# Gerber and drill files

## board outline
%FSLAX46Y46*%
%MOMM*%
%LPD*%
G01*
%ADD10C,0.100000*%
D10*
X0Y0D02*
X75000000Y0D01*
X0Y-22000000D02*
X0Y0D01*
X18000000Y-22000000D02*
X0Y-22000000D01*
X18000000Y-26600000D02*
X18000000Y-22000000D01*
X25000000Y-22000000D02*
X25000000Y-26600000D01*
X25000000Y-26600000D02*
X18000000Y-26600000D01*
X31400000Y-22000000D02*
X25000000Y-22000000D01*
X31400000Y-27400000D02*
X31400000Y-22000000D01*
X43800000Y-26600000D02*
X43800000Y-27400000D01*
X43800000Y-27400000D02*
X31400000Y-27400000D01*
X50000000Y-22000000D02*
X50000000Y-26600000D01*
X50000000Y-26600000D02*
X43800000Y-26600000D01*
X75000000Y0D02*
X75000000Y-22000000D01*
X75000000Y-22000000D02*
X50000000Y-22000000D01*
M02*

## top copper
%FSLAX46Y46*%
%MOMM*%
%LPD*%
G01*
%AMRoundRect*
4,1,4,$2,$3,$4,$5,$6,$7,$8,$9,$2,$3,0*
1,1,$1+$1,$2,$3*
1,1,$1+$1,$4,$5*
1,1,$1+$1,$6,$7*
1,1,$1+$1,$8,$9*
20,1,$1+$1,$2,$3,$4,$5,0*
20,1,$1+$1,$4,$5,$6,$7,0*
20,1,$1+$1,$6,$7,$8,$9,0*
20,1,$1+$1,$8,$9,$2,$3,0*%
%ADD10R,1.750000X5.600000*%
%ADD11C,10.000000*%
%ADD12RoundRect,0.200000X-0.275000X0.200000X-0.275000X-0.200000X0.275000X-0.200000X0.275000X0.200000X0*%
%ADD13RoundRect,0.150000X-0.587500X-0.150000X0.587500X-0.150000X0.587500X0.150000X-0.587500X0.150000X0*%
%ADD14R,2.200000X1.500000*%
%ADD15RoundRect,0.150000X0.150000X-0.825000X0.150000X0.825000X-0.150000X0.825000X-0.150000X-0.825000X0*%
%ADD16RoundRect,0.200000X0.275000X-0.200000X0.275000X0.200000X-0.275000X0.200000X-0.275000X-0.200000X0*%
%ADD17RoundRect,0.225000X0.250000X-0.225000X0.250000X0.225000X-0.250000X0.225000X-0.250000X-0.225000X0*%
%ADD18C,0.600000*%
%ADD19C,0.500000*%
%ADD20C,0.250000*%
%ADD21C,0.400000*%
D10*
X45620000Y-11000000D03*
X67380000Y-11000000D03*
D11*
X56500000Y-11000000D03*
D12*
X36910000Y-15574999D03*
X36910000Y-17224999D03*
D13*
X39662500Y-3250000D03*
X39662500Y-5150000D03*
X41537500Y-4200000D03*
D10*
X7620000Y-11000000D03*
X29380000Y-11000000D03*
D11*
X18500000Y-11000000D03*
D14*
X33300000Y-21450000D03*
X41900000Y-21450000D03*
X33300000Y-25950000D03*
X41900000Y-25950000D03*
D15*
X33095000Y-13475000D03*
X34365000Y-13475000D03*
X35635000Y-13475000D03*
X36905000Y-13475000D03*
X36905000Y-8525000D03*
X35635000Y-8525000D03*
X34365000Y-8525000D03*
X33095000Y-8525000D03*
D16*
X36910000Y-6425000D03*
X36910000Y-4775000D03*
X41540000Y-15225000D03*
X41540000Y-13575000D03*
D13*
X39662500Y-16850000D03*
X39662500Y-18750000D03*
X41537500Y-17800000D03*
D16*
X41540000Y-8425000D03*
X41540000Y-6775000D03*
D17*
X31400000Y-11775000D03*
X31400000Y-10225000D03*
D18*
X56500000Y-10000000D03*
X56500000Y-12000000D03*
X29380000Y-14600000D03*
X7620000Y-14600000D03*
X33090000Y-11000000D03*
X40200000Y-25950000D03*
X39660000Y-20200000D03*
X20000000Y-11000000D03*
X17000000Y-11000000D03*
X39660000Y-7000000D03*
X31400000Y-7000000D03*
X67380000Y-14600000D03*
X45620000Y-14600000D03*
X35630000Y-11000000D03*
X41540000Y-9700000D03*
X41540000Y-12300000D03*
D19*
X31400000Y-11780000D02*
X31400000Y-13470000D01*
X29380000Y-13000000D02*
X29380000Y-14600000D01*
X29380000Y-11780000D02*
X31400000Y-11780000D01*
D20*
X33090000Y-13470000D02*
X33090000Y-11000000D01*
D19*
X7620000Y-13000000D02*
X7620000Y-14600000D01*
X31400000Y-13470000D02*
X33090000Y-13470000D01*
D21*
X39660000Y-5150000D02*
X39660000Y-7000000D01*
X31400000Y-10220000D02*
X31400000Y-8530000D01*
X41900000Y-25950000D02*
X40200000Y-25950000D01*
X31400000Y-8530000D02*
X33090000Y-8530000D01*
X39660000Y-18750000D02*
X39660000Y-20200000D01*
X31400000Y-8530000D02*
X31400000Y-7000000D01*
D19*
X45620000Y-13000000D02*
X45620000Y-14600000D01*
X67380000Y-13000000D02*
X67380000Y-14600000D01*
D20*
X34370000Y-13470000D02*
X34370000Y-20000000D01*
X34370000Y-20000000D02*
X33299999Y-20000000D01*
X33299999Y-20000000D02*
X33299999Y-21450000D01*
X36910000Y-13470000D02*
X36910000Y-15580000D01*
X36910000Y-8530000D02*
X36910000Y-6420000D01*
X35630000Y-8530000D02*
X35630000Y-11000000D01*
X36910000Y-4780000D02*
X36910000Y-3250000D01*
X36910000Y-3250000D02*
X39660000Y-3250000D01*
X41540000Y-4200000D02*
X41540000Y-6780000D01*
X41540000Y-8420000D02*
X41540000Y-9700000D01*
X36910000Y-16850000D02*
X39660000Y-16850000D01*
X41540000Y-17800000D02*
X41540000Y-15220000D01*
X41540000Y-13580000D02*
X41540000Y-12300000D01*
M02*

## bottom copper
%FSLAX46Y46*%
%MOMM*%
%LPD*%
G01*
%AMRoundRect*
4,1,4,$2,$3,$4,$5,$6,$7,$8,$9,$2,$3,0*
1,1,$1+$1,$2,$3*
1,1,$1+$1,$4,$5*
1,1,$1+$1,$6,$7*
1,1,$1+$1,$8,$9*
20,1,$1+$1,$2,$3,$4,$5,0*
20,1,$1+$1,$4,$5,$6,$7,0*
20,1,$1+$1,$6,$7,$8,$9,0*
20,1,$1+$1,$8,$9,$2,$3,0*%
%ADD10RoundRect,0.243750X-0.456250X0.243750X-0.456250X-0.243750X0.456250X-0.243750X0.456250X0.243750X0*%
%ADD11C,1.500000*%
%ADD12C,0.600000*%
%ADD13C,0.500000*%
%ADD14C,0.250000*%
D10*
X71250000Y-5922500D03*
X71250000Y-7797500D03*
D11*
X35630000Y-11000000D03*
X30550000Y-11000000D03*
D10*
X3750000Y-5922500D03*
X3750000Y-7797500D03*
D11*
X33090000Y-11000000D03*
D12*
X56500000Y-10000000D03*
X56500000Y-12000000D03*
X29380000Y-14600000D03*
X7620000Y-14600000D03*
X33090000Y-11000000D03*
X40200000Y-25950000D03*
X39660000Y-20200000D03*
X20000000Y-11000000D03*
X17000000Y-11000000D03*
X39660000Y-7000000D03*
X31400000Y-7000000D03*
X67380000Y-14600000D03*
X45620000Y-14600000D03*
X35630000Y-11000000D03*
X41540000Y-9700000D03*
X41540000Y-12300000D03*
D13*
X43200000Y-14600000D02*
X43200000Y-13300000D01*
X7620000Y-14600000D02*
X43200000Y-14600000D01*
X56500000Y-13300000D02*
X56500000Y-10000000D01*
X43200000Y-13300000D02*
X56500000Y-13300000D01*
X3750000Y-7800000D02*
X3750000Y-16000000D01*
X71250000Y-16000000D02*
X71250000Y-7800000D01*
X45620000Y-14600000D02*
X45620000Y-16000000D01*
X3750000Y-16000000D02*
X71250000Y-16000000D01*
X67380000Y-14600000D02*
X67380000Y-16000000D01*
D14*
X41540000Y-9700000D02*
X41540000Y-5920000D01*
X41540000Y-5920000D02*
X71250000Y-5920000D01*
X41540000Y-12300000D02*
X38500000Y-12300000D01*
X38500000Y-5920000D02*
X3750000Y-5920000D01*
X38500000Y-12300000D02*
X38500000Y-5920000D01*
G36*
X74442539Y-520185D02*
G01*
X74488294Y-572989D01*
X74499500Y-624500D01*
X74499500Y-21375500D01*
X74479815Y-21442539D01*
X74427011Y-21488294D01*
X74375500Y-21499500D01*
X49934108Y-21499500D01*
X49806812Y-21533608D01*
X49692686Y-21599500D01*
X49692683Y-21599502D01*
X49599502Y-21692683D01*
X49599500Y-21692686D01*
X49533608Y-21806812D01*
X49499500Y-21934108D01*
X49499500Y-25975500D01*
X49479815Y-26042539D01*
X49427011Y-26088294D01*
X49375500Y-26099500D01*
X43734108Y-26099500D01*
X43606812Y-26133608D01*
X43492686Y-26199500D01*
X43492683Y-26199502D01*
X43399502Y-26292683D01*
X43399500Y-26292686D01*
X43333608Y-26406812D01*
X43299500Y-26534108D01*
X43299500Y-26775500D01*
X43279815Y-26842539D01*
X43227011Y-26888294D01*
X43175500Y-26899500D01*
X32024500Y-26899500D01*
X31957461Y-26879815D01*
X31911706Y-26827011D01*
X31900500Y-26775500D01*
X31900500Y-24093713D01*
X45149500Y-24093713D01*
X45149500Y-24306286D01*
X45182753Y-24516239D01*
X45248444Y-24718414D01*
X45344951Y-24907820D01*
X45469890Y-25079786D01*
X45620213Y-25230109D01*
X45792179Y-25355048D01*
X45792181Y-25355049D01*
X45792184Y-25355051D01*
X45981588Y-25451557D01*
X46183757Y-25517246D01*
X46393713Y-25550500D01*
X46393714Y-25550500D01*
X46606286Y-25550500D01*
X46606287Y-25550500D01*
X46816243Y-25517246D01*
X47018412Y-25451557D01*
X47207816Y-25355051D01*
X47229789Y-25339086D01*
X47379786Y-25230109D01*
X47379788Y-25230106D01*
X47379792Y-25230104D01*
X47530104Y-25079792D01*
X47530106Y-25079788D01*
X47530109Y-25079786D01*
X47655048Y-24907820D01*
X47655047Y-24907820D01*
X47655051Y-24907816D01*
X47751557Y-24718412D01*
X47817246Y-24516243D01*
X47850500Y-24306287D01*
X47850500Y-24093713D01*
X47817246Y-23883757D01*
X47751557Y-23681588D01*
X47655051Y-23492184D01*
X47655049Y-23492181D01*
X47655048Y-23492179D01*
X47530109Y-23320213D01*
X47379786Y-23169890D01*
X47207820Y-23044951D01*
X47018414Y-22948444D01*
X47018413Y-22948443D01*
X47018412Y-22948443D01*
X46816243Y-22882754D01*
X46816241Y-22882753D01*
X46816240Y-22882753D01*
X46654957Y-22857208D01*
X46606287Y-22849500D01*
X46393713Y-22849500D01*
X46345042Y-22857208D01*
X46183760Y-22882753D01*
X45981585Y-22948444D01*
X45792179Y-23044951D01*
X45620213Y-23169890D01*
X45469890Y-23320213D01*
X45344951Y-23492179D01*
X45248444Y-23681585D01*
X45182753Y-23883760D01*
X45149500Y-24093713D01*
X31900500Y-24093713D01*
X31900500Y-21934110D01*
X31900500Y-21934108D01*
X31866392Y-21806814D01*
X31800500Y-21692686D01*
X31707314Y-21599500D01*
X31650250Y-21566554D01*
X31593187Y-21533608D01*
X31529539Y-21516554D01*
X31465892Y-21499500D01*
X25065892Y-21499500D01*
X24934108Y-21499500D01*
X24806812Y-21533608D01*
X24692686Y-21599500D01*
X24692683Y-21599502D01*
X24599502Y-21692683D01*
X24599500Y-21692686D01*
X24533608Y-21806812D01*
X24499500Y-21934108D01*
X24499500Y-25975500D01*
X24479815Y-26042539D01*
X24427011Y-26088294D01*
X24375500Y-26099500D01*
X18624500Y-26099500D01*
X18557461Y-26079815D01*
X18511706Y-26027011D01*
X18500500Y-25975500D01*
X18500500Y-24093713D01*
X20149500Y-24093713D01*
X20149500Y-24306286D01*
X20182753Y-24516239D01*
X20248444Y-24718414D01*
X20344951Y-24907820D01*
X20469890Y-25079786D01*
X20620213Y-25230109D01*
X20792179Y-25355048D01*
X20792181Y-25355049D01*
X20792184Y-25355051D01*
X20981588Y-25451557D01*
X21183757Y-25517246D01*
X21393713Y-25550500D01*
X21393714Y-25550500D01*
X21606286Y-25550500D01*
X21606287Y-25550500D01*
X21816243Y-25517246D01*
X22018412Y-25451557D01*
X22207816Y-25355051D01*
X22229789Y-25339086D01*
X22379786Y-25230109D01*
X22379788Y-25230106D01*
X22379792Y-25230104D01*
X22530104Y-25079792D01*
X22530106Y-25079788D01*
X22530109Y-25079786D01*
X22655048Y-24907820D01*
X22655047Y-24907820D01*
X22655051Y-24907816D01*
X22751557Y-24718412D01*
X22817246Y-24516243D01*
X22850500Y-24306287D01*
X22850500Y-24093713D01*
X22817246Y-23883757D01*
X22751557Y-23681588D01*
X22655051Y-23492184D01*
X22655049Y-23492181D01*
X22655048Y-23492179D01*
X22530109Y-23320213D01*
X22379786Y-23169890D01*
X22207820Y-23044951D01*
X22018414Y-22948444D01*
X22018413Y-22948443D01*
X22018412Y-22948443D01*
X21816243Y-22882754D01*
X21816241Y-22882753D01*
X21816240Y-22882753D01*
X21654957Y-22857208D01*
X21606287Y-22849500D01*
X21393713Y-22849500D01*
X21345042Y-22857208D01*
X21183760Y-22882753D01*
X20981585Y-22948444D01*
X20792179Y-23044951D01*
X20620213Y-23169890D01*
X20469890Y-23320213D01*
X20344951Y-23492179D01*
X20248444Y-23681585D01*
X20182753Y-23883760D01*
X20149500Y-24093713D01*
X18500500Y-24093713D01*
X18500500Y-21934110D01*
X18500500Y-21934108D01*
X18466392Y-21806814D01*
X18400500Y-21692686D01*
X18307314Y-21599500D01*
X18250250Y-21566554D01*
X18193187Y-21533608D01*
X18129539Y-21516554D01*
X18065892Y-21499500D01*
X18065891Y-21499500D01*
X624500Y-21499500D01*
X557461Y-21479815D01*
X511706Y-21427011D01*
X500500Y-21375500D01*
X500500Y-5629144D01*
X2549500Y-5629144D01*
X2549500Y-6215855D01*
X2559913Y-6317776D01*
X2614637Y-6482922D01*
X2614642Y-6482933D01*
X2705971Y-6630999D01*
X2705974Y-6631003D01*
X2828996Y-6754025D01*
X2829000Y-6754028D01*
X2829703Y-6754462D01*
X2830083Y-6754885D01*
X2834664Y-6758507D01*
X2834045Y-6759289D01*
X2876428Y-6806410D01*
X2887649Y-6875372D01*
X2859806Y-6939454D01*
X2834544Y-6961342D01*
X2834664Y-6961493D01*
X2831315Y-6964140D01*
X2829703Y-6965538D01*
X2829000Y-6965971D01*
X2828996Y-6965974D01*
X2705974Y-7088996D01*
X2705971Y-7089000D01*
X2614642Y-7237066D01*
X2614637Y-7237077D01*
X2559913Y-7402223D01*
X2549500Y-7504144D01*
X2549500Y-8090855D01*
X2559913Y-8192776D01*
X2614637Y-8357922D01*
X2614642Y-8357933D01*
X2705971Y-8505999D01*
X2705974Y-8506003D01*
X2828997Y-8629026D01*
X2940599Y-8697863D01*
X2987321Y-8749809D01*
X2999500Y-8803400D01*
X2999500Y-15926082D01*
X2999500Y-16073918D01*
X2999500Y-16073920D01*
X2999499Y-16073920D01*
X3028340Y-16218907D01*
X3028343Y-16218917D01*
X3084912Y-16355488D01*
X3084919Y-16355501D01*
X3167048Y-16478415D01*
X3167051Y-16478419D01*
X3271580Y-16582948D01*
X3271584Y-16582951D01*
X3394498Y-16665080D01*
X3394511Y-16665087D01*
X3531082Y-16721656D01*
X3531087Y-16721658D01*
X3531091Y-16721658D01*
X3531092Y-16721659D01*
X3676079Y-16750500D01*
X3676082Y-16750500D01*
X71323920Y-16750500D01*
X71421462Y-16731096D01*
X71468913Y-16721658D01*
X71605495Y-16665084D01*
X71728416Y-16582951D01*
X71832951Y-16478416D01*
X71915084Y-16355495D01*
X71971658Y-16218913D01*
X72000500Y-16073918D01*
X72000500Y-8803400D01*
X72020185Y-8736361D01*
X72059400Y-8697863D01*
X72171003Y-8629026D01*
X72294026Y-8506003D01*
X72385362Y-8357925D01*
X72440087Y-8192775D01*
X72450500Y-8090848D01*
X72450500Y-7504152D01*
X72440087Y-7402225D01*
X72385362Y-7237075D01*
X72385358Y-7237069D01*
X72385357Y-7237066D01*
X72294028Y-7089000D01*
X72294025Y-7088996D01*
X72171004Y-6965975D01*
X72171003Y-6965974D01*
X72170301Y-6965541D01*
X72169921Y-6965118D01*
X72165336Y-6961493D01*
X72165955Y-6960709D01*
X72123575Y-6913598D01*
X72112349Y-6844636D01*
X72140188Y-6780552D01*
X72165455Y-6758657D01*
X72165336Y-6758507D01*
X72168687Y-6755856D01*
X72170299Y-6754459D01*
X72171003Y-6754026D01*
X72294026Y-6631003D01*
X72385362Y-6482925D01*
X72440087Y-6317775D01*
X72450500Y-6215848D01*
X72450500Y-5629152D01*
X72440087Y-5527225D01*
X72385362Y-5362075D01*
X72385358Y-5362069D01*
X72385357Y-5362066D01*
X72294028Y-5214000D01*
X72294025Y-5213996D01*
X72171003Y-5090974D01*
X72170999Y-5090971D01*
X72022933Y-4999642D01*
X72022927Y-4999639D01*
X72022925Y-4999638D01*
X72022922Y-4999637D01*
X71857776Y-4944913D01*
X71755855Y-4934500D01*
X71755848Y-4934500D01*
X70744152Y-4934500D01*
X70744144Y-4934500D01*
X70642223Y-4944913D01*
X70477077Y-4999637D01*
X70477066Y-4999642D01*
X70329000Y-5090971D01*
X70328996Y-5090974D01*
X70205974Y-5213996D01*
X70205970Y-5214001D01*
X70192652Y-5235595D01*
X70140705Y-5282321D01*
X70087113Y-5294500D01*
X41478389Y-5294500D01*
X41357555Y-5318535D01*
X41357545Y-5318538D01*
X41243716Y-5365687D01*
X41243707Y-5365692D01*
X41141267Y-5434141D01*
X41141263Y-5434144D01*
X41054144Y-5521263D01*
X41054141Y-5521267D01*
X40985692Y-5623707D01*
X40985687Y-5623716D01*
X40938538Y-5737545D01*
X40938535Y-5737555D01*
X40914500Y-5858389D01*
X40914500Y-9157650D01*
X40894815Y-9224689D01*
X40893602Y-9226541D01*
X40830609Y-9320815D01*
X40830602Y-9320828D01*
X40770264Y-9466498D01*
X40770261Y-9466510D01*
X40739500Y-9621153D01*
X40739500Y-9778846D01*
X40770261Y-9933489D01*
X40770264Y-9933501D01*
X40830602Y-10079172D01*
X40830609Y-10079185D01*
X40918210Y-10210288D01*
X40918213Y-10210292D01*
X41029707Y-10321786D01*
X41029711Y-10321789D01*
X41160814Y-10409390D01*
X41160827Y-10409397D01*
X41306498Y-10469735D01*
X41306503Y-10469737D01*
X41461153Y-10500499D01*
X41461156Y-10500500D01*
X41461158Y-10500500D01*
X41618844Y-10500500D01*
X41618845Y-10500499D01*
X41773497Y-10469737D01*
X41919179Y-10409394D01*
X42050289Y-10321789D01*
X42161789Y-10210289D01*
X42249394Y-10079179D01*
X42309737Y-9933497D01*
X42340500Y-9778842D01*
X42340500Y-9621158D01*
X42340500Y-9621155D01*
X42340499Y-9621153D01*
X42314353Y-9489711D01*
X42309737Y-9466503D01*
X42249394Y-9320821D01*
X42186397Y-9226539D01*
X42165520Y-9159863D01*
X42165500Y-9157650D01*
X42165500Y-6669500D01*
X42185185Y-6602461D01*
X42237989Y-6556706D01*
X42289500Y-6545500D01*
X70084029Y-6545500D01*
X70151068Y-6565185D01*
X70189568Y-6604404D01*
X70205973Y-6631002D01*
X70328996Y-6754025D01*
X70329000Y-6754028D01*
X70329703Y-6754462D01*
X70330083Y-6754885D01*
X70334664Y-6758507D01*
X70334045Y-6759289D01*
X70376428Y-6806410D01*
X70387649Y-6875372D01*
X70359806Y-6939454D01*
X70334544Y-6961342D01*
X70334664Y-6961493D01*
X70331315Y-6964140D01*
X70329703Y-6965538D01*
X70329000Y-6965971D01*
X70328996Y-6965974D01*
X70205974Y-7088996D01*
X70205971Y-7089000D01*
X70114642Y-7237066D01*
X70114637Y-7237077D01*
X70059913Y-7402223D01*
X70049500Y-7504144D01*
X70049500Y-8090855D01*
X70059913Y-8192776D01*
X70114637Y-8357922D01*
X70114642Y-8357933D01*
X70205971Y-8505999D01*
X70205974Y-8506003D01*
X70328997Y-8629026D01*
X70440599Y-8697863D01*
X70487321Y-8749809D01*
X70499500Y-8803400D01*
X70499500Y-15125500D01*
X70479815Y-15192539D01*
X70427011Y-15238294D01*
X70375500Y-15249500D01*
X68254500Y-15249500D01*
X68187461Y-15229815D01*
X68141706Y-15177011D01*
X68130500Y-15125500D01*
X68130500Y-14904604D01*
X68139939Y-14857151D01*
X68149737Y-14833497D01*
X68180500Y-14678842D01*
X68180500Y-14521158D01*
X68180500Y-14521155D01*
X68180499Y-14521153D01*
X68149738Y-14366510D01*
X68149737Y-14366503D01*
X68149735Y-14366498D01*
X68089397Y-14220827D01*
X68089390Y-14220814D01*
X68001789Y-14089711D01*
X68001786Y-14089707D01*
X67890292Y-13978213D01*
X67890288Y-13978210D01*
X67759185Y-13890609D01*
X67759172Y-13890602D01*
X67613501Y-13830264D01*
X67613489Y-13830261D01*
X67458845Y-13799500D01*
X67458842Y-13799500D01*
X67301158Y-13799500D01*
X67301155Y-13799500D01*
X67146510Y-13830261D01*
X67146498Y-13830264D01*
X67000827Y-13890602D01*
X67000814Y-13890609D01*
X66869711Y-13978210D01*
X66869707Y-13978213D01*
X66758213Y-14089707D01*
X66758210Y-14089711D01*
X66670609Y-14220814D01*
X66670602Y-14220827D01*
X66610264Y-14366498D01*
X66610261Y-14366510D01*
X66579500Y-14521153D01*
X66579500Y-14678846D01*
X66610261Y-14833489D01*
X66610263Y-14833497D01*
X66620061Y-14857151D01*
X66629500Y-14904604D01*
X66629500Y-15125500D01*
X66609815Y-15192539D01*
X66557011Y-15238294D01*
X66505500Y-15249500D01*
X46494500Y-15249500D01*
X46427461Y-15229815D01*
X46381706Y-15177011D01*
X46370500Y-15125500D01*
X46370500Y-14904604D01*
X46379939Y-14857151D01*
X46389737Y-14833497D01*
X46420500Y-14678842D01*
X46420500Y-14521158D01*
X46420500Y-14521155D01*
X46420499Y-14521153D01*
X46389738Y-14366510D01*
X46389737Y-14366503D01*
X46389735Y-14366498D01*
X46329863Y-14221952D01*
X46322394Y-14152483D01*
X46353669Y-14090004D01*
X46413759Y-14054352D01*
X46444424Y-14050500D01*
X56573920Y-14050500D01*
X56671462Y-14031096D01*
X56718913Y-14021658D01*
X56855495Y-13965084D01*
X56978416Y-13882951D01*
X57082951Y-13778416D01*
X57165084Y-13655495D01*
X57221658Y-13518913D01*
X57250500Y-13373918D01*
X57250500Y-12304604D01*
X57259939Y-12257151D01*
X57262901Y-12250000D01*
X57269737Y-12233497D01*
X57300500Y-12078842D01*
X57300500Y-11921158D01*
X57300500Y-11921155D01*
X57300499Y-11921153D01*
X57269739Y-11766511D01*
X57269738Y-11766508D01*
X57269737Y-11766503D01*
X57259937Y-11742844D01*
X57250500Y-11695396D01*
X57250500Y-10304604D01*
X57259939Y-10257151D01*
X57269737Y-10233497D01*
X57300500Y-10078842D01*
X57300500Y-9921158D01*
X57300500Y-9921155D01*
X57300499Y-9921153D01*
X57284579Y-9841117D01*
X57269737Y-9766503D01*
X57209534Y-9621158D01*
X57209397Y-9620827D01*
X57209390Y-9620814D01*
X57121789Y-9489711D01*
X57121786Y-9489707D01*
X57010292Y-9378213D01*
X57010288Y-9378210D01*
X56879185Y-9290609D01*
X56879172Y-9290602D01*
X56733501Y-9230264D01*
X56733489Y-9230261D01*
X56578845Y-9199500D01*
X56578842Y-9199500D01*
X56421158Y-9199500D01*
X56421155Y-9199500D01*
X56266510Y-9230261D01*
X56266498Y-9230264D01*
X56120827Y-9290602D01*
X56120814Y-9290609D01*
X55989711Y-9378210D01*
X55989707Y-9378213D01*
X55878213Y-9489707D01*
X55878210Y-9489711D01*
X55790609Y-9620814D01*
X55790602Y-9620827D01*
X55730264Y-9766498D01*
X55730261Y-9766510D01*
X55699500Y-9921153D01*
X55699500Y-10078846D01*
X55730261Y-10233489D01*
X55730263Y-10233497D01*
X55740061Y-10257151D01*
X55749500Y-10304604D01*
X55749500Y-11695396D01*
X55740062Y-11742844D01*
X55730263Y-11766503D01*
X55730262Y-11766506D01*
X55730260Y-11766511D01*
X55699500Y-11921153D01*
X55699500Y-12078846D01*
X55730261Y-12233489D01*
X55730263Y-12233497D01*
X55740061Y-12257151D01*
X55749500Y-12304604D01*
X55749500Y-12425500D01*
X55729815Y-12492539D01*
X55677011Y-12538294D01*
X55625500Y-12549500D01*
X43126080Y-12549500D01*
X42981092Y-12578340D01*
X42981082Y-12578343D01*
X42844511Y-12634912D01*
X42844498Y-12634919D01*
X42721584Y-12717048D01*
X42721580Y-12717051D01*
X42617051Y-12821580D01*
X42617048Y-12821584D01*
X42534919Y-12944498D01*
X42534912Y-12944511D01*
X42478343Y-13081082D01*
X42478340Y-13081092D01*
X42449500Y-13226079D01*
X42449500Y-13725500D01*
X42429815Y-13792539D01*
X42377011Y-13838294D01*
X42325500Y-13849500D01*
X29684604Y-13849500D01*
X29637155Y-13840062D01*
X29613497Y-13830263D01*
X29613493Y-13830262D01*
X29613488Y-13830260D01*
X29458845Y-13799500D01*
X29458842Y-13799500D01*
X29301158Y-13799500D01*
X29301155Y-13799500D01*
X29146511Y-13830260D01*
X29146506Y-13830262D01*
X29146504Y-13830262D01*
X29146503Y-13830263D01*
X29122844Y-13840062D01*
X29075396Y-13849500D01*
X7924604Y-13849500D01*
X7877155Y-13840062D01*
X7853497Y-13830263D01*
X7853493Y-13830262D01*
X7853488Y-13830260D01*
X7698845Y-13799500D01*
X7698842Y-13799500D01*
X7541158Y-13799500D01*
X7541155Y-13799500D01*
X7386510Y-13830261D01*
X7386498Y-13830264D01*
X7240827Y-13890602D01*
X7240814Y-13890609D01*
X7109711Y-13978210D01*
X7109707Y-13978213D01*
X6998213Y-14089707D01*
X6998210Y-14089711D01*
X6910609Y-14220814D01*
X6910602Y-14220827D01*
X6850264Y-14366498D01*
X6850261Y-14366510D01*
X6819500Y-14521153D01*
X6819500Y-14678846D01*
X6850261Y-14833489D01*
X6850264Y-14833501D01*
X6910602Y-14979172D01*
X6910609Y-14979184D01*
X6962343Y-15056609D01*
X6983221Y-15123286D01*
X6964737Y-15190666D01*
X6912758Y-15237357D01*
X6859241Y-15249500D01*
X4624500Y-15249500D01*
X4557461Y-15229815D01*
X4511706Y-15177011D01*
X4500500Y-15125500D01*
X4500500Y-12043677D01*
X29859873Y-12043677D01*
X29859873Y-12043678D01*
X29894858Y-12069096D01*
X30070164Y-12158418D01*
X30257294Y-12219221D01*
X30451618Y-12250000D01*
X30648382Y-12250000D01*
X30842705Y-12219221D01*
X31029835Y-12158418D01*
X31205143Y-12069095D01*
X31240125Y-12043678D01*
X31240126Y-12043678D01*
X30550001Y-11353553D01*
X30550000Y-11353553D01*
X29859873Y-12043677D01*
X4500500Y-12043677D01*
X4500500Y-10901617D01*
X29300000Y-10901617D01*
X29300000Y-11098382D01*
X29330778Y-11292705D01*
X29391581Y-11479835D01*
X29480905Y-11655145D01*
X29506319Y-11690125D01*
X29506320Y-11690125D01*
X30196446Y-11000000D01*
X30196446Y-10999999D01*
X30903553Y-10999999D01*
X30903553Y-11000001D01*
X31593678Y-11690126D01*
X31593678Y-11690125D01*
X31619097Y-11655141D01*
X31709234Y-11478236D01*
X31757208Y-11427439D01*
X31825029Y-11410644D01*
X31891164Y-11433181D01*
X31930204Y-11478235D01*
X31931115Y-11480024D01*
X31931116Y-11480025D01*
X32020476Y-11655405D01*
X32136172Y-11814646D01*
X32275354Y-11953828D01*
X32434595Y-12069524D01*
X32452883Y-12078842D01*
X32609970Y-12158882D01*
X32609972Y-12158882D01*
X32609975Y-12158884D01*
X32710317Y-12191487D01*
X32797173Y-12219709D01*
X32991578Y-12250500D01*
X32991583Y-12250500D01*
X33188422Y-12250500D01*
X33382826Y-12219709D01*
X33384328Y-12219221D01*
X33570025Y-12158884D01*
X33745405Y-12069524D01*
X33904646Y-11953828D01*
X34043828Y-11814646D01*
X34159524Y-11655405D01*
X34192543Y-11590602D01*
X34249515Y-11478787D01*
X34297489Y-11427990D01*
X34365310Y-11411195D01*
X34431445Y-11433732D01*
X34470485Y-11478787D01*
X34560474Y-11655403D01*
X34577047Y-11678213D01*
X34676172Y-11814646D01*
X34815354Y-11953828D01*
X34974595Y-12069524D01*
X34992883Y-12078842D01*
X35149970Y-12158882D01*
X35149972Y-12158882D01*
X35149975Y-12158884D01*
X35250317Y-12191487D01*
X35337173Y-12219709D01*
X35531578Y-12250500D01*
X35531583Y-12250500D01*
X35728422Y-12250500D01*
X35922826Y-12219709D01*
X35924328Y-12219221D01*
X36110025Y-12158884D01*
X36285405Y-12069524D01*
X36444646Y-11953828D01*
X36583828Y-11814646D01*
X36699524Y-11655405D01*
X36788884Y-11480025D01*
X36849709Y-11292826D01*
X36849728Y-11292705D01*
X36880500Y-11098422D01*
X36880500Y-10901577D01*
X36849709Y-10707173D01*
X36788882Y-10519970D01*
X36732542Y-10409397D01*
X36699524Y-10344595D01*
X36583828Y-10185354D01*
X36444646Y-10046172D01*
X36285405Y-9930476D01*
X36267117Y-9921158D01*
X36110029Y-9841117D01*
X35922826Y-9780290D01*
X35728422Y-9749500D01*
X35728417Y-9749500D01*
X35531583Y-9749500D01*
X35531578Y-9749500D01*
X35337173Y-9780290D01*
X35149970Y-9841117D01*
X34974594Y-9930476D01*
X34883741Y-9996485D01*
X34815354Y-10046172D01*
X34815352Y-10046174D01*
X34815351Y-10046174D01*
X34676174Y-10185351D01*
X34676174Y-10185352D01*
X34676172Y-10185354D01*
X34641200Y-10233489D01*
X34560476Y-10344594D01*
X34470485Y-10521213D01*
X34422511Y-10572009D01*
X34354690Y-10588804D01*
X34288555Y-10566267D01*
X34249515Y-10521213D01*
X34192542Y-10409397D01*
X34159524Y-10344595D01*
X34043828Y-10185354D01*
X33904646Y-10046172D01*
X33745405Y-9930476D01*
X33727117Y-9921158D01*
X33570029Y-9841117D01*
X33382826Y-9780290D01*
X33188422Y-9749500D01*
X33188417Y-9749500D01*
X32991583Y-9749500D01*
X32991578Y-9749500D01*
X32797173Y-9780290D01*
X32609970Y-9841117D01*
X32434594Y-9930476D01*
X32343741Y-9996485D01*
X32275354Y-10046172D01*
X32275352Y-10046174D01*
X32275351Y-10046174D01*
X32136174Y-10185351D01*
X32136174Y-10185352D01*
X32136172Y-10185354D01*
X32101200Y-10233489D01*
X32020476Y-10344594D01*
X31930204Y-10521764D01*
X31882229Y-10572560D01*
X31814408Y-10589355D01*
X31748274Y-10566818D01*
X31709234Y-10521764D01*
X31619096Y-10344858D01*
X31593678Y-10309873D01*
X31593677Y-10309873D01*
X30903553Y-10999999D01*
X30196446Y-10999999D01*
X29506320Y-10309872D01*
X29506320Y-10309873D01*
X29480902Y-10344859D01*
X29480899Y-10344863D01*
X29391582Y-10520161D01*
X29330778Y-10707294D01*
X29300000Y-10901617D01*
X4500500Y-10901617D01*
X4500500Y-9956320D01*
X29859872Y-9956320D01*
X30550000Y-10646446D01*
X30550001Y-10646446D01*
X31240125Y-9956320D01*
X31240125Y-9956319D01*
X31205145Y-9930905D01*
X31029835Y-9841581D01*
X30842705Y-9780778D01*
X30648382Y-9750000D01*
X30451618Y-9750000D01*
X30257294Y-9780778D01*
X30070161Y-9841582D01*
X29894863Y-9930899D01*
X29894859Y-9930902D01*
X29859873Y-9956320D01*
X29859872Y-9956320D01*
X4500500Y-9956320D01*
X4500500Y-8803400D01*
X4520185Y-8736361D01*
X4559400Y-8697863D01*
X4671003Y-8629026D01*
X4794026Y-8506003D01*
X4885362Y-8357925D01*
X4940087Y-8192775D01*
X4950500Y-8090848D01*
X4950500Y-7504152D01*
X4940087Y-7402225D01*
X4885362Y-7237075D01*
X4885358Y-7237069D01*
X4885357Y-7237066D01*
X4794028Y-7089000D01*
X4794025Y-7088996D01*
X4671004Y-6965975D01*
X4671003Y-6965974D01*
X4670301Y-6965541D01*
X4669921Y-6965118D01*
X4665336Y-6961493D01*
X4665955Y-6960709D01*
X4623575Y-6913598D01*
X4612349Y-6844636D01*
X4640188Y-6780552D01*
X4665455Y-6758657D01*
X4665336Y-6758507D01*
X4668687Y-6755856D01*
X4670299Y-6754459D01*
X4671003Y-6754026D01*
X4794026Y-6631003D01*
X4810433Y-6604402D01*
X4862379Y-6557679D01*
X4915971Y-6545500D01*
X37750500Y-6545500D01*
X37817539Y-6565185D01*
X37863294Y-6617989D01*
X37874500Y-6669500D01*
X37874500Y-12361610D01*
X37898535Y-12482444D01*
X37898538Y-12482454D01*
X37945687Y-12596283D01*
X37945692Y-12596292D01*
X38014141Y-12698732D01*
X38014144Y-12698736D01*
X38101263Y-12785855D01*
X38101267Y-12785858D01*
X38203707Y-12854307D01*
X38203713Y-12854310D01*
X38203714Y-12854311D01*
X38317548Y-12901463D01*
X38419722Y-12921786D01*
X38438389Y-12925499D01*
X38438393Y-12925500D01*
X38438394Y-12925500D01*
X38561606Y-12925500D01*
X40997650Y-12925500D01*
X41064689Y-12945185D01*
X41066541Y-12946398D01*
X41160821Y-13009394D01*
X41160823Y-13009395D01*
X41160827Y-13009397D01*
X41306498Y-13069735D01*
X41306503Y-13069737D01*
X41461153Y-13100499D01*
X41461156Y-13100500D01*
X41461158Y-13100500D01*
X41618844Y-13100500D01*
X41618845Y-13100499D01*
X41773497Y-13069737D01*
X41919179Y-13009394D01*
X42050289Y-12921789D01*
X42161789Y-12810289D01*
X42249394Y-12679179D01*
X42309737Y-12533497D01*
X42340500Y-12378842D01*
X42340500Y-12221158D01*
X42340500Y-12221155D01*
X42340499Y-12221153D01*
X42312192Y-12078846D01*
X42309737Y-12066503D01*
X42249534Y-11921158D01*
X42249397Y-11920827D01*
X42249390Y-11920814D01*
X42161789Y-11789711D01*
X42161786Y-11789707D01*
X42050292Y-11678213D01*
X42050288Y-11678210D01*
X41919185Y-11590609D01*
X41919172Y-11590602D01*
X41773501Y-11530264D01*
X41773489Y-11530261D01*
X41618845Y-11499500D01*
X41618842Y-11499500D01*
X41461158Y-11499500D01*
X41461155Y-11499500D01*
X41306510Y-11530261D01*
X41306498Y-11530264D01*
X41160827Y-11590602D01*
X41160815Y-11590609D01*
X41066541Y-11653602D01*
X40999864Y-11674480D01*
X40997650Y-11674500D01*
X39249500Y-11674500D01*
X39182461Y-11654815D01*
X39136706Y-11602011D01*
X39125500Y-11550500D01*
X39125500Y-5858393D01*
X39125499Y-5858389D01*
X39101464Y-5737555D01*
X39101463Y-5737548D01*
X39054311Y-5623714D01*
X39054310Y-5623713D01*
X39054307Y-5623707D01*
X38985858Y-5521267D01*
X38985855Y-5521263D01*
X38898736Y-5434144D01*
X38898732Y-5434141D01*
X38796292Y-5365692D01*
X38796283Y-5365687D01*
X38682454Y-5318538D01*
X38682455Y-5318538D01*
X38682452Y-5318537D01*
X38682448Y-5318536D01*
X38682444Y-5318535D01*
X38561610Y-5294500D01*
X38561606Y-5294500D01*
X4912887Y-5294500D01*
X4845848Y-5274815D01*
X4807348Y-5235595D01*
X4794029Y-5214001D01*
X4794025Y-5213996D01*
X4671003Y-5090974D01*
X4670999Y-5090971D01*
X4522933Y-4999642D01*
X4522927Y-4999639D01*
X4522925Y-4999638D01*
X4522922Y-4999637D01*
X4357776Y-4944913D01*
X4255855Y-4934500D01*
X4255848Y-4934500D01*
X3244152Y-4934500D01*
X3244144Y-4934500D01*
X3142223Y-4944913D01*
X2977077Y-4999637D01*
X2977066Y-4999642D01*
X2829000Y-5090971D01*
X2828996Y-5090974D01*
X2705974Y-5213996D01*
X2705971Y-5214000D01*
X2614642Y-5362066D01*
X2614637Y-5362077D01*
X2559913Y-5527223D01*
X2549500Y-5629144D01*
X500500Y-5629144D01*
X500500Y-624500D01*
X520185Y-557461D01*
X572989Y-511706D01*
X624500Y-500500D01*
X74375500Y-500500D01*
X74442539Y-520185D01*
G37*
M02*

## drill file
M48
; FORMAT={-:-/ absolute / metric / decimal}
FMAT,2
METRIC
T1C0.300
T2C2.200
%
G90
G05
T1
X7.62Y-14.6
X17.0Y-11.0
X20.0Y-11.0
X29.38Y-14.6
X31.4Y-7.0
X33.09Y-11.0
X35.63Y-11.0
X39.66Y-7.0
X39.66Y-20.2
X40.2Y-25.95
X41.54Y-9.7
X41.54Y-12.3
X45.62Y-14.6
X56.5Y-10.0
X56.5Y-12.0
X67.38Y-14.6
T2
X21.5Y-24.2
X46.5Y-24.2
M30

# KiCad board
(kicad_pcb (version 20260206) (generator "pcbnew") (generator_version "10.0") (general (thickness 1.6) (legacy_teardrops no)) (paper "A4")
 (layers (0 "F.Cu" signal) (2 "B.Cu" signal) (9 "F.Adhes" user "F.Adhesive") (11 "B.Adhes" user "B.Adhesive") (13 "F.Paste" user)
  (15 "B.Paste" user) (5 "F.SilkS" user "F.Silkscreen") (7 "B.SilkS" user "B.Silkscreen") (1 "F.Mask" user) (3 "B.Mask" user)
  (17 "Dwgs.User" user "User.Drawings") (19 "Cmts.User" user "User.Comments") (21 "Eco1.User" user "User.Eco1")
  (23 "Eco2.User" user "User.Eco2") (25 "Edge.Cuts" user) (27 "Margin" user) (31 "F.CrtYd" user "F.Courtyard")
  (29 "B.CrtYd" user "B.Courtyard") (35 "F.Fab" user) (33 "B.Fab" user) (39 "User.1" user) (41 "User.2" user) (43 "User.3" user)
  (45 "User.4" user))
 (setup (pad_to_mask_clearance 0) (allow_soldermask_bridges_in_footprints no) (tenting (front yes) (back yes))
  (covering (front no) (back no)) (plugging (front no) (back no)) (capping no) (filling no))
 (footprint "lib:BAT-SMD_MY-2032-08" (layer "F.Cu") (at 56.5 11)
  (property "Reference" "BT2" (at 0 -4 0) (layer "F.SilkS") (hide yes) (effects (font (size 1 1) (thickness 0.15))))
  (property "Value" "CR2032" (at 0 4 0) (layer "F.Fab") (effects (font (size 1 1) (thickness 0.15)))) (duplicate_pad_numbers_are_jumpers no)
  (pad "1" smd rect (at -10.88 0) (size 1.75 5.6) (layers "F.Cu" "F.Mask" "F.Paste") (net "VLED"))
  (pad "1" smd rect (at 10.88 0) (size 1.75 5.6) (layers "F.Cu" "F.Mask" "F.Paste") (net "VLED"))
  (pad "2" smd circle (at 0 0) (size 10 10) (layers "F.Cu" "F.Mask" "F.Paste") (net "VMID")))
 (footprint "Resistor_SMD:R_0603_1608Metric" (layer "F.Cu") (at 36.91 16.399999 -90)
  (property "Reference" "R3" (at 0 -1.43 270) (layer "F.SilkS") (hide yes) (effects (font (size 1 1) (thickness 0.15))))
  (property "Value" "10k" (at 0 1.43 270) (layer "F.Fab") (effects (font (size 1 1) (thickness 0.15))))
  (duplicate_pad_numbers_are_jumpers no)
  (pad "1" smd roundrect (at -0.825 0 270) (size 0.8 0.95) (layers "F.Cu" "F.Mask" "F.Paste") (roundrect_rratio 0.25) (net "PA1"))
  (pad "2" smd roundrect (at 0.825 0 270) (size 0.8 0.95) (layers "F.Cu" "F.Mask" "F.Paste") (roundrect_rratio 0.25) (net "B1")))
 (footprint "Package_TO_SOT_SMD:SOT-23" (layer "F.Cu") (at 40.6 4.2)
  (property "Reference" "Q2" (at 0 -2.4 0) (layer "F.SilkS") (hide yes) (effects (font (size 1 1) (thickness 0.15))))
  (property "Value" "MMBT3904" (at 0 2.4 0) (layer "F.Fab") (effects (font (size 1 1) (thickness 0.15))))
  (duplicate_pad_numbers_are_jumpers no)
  (pad "1" smd roundrect (at -0.9375 -0.95) (size 1.475 0.6) (layers "F.Cu" "F.Mask" "F.Paste") (roundrect_rratio 0.25) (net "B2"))
  (pad "2" smd roundrect (at -0.9375 0.95) (size 1.475 0.6) (layers "F.Cu" "F.Mask" "F.Paste") (roundrect_rratio 0.25) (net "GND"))
  (pad "3" smd roundrect (at 0.9375 0) (size 1.475 0.6) (layers "F.Cu" "F.Mask" "F.Paste") (roundrect_rratio 0.25) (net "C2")))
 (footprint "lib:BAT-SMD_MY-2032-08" (layer "F.Cu") (at 18.5 11)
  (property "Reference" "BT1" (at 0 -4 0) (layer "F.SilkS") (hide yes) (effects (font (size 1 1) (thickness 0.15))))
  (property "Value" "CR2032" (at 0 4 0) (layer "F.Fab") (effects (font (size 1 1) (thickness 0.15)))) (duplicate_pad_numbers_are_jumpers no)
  (pad "1" smd rect (at -10.88 0) (size 1.75 5.6) (layers "F.Cu" "F.Mask" "F.Paste") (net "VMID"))
  (pad "1" smd rect (at 10.88 0) (size 1.75 5.6) (layers "F.Cu" "F.Mask" "F.Paste") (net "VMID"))
  (pad "2" smd circle (at 0 0) (size 10 10) (layers "F.Cu" "F.Mask" "F.Paste") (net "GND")))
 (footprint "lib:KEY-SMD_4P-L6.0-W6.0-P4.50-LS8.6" (layer "F.Cu") (at 37.6 23.7)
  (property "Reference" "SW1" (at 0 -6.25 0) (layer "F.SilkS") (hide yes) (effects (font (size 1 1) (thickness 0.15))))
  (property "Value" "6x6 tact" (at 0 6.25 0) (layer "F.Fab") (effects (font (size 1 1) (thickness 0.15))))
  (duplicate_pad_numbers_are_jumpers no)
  (pad "1" smd rect (at -4.3 -2.25) (size 2.2 1.5) (layers "F.Cu" "F.Mask" "F.Paste") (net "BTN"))
  (pad "2" smd rect (at 4.3 -2.25) (size 2.2 1.5) (layers "F.Cu" "F.Mask" "F.Paste"))
  (pad "3" smd rect (at -4.3 2.25) (size 2.2 1.5) (layers "F.Cu" "F.Mask" "F.Paste"))
  (pad "4" smd rect (at 4.3 2.25) (size 2.2 1.5) (layers "F.Cu" "F.Mask" "F.Paste") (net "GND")))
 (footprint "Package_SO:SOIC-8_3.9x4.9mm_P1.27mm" (layer "F.Cu") (at 35 11 90)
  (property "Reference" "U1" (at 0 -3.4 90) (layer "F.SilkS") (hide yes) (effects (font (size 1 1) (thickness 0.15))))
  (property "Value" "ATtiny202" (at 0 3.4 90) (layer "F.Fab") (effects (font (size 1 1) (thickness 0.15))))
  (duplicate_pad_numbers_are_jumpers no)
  (pad "1" smd roundrect (at -2.475 -1.905 90) (size 1.95 0.6) (layers "F.Cu" "F.Mask" "F.Paste") (roundrect_rratio 0.25) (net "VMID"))
  (pad "2" smd roundrect (at -2.475 -0.635 90) (size 1.95 0.6) (layers "F.Cu" "F.Mask" "F.Paste") (roundrect_rratio 0.25) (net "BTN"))
  (pad "3" smd roundrect (at -2.475 0.635 90) (size 1.95 0.6) (layers "F.Cu" "F.Mask" "F.Paste") (roundrect_rratio 0.25))
  (pad "4" smd roundrect (at -2.475 1.905 90) (size 1.95 0.6) (layers "F.Cu" "F.Mask" "F.Paste") (roundrect_rratio 0.25) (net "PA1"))
  (pad "5" smd roundrect (at 2.475 1.905 90) (size 1.95 0.6) (layers "F.Cu" "F.Mask" "F.Paste") (roundrect_rratio 0.25) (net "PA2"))
  (pad "6" smd roundrect (at 2.475 0.635 90) (size 1.95 0.6) (layers "F.Cu" "F.Mask" "F.Paste") (roundrect_rratio 0.25) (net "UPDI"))
  (pad "7" smd roundrect (at 2.475 -0.635 90) (size 1.95 0.6) (layers "F.Cu" "F.Mask" "F.Paste") (roundrect_rratio 0.25))
  (pad "8" smd roundrect (at 2.475 -1.905 90) (size 1.95 0.6) (layers "F.Cu" "F.Mask" "F.Paste") (roundrect_rratio 0.25) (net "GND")))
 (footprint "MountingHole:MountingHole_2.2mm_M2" (layer "F.Cu") (at 21.5 24.2)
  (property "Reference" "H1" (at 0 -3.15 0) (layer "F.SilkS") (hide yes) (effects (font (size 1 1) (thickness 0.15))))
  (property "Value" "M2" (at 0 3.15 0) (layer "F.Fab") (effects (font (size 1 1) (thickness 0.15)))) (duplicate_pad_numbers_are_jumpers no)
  (pad "" np_thru_hole circle (at 0 0) (size 2.2 2.2) (drill 2.2) (layers "*.Cu" "*.Mask")))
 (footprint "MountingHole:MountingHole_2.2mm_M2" (layer "F.Cu") (at 46.5 24.2)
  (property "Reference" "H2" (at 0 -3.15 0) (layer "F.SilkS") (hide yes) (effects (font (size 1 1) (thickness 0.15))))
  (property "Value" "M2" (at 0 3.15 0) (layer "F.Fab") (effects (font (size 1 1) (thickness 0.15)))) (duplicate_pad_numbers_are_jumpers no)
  (pad "" np_thru_hole circle (at 0 0) (size 2.2 2.2) (drill 2.2) (layers "*.Cu" "*.Mask")))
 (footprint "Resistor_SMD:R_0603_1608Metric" (layer "F.Cu") (at 36.91 5.6 90)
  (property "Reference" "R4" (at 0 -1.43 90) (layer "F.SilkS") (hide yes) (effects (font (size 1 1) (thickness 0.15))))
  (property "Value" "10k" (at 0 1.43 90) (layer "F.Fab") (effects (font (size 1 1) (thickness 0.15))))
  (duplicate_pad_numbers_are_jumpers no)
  (pad "1" smd roundrect (at -0.825 0 90) (size 0.8 0.95) (layers "F.Cu" "F.Mask" "F.Paste") (roundrect_rratio 0.25) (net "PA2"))
  (pad "2" smd roundrect (at 0.825 0 90) (size 0.8 0.95) (layers "F.Cu" "F.Mask" "F.Paste") (roundrect_rratio 0.25) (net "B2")))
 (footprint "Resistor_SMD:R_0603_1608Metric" (layer "F.Cu") (at 41.54 14.4 90)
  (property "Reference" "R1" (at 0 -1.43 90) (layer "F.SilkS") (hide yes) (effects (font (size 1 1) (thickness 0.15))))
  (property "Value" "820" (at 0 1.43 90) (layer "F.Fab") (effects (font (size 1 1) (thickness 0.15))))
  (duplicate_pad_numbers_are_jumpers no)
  (pad "1" smd roundrect (at -0.825 0 90) (size 0.8 0.95) (layers "F.Cu" "F.Mask" "F.Paste") (roundrect_rratio 0.25) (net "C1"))
  (pad "2" smd roundrect (at 0.825 0 90) (size 0.8 0.95) (layers "F.Cu" "F.Mask" "F.Paste") (roundrect_rratio 0.25) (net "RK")))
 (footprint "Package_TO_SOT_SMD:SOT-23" (layer "F.Cu") (at 40.6 17.8)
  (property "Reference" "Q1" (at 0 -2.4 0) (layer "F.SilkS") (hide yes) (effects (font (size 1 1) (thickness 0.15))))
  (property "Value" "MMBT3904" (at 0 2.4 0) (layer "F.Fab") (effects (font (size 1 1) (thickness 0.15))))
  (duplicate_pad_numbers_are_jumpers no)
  (pad "1" smd roundrect (at -0.9375 -0.95) (size 1.475 0.6) (layers "F.Cu" "F.Mask" "F.Paste") (roundrect_rratio 0.25) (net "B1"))
  (pad "2" smd roundrect (at -0.9375 0.95) (size 1.475 0.6) (layers "F.Cu" "F.Mask" "F.Paste") (roundrect_rratio 0.25) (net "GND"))
  (pad "3" smd roundrect (at 0.9375 0) (size 1.475 0.6) (layers "F.Cu" "F.Mask" "F.Paste") (roundrect_rratio 0.25) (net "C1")))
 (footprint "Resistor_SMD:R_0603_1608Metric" (layer "F.Cu") (at 41.54 7.6 90)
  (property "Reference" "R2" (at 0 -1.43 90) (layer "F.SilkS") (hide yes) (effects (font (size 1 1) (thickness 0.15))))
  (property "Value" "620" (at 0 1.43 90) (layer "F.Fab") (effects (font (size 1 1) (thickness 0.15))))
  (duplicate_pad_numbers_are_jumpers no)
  (pad "1" smd roundrect (at -0.825 0 90) (size 0.8 0.95) (layers "F.Cu" "F.Mask" "F.Paste") (roundrect_rratio 0.25) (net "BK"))
  (pad "2" smd roundrect (at 0.825 0 90) (size 0.8 0.95) (layers "F.Cu" "F.Mask" "F.Paste") (roundrect_rratio 0.25) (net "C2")))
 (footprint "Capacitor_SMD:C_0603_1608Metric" (layer "F.Cu") (at 31.4 11 90)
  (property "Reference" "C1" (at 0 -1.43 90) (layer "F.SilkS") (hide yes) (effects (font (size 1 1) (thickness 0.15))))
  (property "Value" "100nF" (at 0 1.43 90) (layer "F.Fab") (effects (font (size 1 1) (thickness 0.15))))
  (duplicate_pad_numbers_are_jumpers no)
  (pad "1" smd roundrect (at -0.775 0 90) (size 0.9 0.95) (layers "F.Cu" "F.Mask" "F.Paste") (roundrect_rratio 0.25) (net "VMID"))
  (pad "2" smd roundrect (at 0.775 0 90) (size 0.9 0.95) (layers "F.Cu" "F.Mask" "F.Paste") (roundrect_rratio 0.25) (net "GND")))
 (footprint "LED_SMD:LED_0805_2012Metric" (layer "B.Cu") (at 71.25 6.86 -90)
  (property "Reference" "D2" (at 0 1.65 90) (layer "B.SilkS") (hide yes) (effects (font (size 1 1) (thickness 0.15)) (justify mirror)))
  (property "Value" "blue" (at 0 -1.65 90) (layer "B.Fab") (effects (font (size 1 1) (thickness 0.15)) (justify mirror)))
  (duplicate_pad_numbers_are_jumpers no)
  (pad "1" smd roundrect (at -0.9375 0 270) (size 0.975 1.4) (layers "B.Cu" "B.Mask" "B.Paste") (roundrect_rratio 0.25) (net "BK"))
  (pad "2" smd roundrect (at 0.9375 0 270) (size 0.975 1.4) (layers "B.Cu" "B.Mask" "B.Paste") (roundrect_rratio 0.25) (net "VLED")))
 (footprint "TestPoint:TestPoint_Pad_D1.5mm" (layer "B.Cu") (at 35.63 11)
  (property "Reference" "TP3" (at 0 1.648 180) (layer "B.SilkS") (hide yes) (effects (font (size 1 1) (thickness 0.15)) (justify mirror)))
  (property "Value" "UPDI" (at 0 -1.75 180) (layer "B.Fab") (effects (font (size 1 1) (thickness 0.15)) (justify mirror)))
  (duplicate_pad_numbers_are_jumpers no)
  (pad "1" smd circle (at 0 0) (size 1.5 1.5) (layers "B.Cu" "B.Mask") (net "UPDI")))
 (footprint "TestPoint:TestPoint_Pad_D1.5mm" (layer "B.Cu") (at 30.55 11)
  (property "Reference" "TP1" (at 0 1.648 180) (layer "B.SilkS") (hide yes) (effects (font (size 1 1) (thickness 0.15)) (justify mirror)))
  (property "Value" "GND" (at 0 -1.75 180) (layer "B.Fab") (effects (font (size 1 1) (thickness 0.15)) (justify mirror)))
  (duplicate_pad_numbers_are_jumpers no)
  (pad "1" smd circle (at 0 0) (size 1.5 1.5) (layers "B.Cu" "B.Mask") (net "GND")))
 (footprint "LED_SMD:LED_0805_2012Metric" (layer "B.Cu") (at 3.75 6.86 -90)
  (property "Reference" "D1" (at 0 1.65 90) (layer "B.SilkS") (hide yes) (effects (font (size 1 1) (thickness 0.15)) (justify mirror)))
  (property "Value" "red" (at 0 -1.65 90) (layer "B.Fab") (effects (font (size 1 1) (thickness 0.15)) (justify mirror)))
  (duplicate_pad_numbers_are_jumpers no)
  (pad "1" smd roundrect (at -0.9375 0 270) (size 0.975 1.4) (layers "B.Cu" "B.Mask" "B.Paste") (roundrect_rratio 0.25) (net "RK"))
  (pad "2" smd roundrect (at 0.9375 0 270) (size 0.975 1.4) (layers "B.Cu" "B.Mask" "B.Paste") (roundrect_rratio 0.25) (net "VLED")))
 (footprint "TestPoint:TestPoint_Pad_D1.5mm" (layer "B.Cu") (at 33.09 11)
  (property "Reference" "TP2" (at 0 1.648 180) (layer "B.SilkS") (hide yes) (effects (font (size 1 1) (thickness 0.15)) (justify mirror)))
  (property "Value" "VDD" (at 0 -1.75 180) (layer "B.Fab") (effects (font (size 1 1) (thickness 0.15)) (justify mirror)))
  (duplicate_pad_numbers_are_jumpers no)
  (pad "1" smd circle (at 0 0) (size 1.5 1.5) (layers "B.Cu" "B.Mask") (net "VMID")))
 (gr_line (start 0 0) (end 75 0) (stroke (width 0.1) (type default)) (layer "Edge.Cuts"))
 (gr_line (start 0 22) (end 0 0) (stroke (width 0.1) (type default)) (layer "Edge.Cuts"))
 (gr_line (start 18 22) (end 0 22) (stroke (width 0.1) (type default)) (layer "Edge.Cuts"))
 (gr_line (start 18 26.6) (end 18 22) (stroke (width 0.1) (type default)) (layer "Edge.Cuts"))
 (gr_line (start 25 22) (end 25 26.6) (stroke (width 0.1) (type default)) (layer "Edge.Cuts"))
 (gr_line (start 25 26.6) (end 18 26.6) (stroke (width 0.1) (type default)) (layer "Edge.Cuts"))
 (gr_line (start 31.4 22) (end 25 22) (stroke (width 0.1) (type default)) (layer "Edge.Cuts"))
 (gr_line (start 31.4 27.4) (end 31.4 22) (stroke (width 0.1) (type default)) (layer "Edge.Cuts"))
 (gr_line (start 43.8 26.6) (end 43.8 27.4) (stroke (width 0.1) (type default)) (layer "Edge.Cuts"))
 (gr_line (start 43.8 27.4) (end 31.4 27.4) (stroke (width 0.1) (type default)) (layer "Edge.Cuts"))
 (gr_line (start 50 22) (end 50 26.6) (stroke (width 0.1) (type default)) (layer "Edge.Cuts"))
 (gr_line (start 50 26.6) (end 43.8 26.6) (stroke (width 0.1) (type default)) (layer "Edge.Cuts"))
 (gr_line (start 75 0) (end 75 22) (stroke (width 0.1) (type default)) (layer "Edge.Cuts"))
 (gr_line (start 75 22) (end 50 22) (stroke (width 0.1) (type default)) (layer "Edge.Cuts"))
 (segment (start 31.4 11.78) (end 31.4 13.47) (width 0.5) (layer "F.Cu") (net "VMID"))
 (segment (start 29.38 13) (end 29.38 14.6) (width 0.5) (layer "F.Cu") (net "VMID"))
 (segment (start 29.38 11.78) (end 31.4 11.78) (width 0.5) (layer "F.Cu") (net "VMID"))
 (segment (start 33.09 13.47) (end 33.09 11) (width 0.25) (layer "F.Cu") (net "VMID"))
 (segment (start 7.62 13) (end 7.62 14.6) (width 0.5) (layer "F.Cu") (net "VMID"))
 (segment (start 31.4 13.47) (end 33.09 13.47) (width 0.5) (layer "F.Cu") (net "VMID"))
 (via (at 56.5 10) (size 0.6) (drill 0.3) (layers "F.Cu" "B.Cu") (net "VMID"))
 (via (at 56.5 12) (size 0.6) (drill 0.3) (layers "F.Cu" "B.Cu") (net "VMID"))
 (via (at 29.38 14.6) (size 0.6) (drill 0.3) (layers "F.Cu" "B.Cu") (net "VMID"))
 (via (at 7.62 14.6) (size 0.6) (drill 0.3) (layers "F.Cu" "B.Cu") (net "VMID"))
 (via (at 33.09 11) (size 0.6) (drill 0.3) (layers "F.Cu" "B.Cu") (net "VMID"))
 (segment (start 43.2 14.6) (end 43.2 13.3) (width 0.5) (layer "B.Cu") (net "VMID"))
 (segment (start 7.62 14.6) (end 43.2 14.6) (width 0.5) (layer "B.Cu") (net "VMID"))
 (segment (start 56.5 13.3) (end 56.5 10) (width 0.5) (layer "B.Cu") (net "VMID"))
 (segment (start 43.2 13.3) (end 56.5 13.3) (width 0.5) (layer "B.Cu") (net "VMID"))
 (segment (start 39.66 5.15) (end 39.66 7) (width 0.4) (layer "F.Cu") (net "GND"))
 (segment (start 31.4 10.22) (end 31.4 8.53) (width 0.4) (layer "F.Cu") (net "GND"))
 (segment (start 41.9 25.95) (end 40.2 25.95) (width 0.4) (layer "F.Cu") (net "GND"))
 (segment (start 31.4 8.53) (end 33.09 8.53) (width 0.4) (layer "F.Cu") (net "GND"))
 (segment (start 39.66 18.75) (end 39.66 20.2) (width 0.4) (layer "F.Cu") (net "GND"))
 (segment (start 31.4 8.53) (end 31.4 7) (width 0.4) (layer "F.Cu") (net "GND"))
 (via (at 40.2 25.95) (size 0.6) (drill 0.3) (layers "F.Cu" "B.Cu") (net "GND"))
 (via (at 39.66 20.2) (size 0.6) (drill 0.3) (layers "F.Cu" "B.Cu") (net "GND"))
 (via (at 20 11) (size 0.6) (drill 0.3) (layers "F.Cu" "B.Cu") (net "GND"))
 (via (at 17 11) (size 0.6) (drill 0.3) (layers "F.Cu" "B.Cu") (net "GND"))
 (via (at 39.66 7) (size 0.6) (drill 0.3) (layers "F.Cu" "B.Cu") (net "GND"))
 (via (at 31.4 7) (size 0.6) (drill 0.3) (layers "F.Cu" "B.Cu") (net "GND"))
 (segment (start 45.62 13) (end 45.62 14.6) (width 0.5) (layer "F.Cu") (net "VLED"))
 (segment (start 67.38 13) (end 67.38 14.6) (width 0.5) (layer "F.Cu") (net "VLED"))
 (via (at 67.38 14.6) (size 0.6) (drill 0.3) (layers "F.Cu" "B.Cu") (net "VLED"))
 (via (at 45.62 14.6) (size 0.6) (drill 0.3) (layers "F.Cu" "B.Cu") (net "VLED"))
 (segment (start 3.75 7.8) (end 3.75 16) (width 0.5) (layer "B.Cu") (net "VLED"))
 (segment (start 71.25 16) (end 71.25 7.8) (width 0.5) (layer "B.Cu") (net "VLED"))
 (segment (start 45.62 14.6) (end 45.62 16) (width 0.5) (layer "B.Cu") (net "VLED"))
 (segment (start 3.75 16) (end 71.25 16) (width 0.5) (layer "B.Cu") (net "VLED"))
 (segment (start 67.38 14.6) (end 67.38 16) (width 0.5) (layer "B.Cu") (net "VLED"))
 (segment (start 34.37 13.47) (end 34.37 20) (width 0.25) (layer "F.Cu") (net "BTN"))
 (segment (start 34.37 20) (end 33.299999 20) (width 0.25) (layer "F.Cu") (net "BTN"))
 (segment (start 33.299999 20) (end 33.299999 21.45) (width 0.25) (layer "F.Cu") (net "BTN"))
 (segment (start 36.91 13.47) (end 36.91 15.58) (width 0.25) (layer "F.Cu") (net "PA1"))
 (segment (start 36.91 8.53) (end 36.91 6.42) (width 0.25) (layer "F.Cu") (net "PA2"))
 (segment (start 35.63 8.53) (end 35.63 11) (width 0.25) (layer "F.Cu") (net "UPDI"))
 (via (at 35.63 11) (size 0.6) (drill 0.3) (layers "F.Cu" "B.Cu") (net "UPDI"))
 (segment (start 36.91 4.78) (end 36.91 3.25) (width 0.25) (layer "F.Cu") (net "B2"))
 (segment (start 36.91 3.25) (end 39.66 3.25) (width 0.25) (layer "F.Cu") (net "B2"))
 (segment (start 41.54 4.2) (end 41.54 6.78) (width 0.25) (layer "F.Cu") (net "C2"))
 (segment (start 41.54 8.42) (end 41.54 9.7) (width 0.25) (layer "F.Cu") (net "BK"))
 (via (at 41.54 9.7) (size 0.6) (drill 0.3) (layers "F.Cu" "B.Cu") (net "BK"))
 (segment (start 41.54 9.7) (end 41.54 5.92) (width 0.25) (layer "B.Cu") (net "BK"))
 (segment (start 41.54 5.92) (end 71.25 5.92) (width 0.25) (layer "B.Cu") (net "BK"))
 (segment (start 36.91 16.85) (end 39.66 16.85) (width 0.25) (layer "F.Cu") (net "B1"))
 (segment (start 41.54 17.8) (end 41.54 15.22) (width 0.25) (layer "F.Cu") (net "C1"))
 (segment (start 41.54 13.58) (end 41.54 12.3) (width 0.25) (layer "F.Cu") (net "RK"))
 (via (at 41.54 12.3) (size 0.6) (drill 0.3) (layers "F.Cu" "B.Cu") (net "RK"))
 (segment (start 41.54 12.3) (end 38.5 12.3) (width 0.25) (layer "B.Cu") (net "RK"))
 (segment (start 38.5 5.92) (end 3.75 5.92) (width 0.25) (layer "B.Cu") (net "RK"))
 (segment (start 38.5 12.3) (end 38.5 5.92) (width 0.25) (layer "B.Cu") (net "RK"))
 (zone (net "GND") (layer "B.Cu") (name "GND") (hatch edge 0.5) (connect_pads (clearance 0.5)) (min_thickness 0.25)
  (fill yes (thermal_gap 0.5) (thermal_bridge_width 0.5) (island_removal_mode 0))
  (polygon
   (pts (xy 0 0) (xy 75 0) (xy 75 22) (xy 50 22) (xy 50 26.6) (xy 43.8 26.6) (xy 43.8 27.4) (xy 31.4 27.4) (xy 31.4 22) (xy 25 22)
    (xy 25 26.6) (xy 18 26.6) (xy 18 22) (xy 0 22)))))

